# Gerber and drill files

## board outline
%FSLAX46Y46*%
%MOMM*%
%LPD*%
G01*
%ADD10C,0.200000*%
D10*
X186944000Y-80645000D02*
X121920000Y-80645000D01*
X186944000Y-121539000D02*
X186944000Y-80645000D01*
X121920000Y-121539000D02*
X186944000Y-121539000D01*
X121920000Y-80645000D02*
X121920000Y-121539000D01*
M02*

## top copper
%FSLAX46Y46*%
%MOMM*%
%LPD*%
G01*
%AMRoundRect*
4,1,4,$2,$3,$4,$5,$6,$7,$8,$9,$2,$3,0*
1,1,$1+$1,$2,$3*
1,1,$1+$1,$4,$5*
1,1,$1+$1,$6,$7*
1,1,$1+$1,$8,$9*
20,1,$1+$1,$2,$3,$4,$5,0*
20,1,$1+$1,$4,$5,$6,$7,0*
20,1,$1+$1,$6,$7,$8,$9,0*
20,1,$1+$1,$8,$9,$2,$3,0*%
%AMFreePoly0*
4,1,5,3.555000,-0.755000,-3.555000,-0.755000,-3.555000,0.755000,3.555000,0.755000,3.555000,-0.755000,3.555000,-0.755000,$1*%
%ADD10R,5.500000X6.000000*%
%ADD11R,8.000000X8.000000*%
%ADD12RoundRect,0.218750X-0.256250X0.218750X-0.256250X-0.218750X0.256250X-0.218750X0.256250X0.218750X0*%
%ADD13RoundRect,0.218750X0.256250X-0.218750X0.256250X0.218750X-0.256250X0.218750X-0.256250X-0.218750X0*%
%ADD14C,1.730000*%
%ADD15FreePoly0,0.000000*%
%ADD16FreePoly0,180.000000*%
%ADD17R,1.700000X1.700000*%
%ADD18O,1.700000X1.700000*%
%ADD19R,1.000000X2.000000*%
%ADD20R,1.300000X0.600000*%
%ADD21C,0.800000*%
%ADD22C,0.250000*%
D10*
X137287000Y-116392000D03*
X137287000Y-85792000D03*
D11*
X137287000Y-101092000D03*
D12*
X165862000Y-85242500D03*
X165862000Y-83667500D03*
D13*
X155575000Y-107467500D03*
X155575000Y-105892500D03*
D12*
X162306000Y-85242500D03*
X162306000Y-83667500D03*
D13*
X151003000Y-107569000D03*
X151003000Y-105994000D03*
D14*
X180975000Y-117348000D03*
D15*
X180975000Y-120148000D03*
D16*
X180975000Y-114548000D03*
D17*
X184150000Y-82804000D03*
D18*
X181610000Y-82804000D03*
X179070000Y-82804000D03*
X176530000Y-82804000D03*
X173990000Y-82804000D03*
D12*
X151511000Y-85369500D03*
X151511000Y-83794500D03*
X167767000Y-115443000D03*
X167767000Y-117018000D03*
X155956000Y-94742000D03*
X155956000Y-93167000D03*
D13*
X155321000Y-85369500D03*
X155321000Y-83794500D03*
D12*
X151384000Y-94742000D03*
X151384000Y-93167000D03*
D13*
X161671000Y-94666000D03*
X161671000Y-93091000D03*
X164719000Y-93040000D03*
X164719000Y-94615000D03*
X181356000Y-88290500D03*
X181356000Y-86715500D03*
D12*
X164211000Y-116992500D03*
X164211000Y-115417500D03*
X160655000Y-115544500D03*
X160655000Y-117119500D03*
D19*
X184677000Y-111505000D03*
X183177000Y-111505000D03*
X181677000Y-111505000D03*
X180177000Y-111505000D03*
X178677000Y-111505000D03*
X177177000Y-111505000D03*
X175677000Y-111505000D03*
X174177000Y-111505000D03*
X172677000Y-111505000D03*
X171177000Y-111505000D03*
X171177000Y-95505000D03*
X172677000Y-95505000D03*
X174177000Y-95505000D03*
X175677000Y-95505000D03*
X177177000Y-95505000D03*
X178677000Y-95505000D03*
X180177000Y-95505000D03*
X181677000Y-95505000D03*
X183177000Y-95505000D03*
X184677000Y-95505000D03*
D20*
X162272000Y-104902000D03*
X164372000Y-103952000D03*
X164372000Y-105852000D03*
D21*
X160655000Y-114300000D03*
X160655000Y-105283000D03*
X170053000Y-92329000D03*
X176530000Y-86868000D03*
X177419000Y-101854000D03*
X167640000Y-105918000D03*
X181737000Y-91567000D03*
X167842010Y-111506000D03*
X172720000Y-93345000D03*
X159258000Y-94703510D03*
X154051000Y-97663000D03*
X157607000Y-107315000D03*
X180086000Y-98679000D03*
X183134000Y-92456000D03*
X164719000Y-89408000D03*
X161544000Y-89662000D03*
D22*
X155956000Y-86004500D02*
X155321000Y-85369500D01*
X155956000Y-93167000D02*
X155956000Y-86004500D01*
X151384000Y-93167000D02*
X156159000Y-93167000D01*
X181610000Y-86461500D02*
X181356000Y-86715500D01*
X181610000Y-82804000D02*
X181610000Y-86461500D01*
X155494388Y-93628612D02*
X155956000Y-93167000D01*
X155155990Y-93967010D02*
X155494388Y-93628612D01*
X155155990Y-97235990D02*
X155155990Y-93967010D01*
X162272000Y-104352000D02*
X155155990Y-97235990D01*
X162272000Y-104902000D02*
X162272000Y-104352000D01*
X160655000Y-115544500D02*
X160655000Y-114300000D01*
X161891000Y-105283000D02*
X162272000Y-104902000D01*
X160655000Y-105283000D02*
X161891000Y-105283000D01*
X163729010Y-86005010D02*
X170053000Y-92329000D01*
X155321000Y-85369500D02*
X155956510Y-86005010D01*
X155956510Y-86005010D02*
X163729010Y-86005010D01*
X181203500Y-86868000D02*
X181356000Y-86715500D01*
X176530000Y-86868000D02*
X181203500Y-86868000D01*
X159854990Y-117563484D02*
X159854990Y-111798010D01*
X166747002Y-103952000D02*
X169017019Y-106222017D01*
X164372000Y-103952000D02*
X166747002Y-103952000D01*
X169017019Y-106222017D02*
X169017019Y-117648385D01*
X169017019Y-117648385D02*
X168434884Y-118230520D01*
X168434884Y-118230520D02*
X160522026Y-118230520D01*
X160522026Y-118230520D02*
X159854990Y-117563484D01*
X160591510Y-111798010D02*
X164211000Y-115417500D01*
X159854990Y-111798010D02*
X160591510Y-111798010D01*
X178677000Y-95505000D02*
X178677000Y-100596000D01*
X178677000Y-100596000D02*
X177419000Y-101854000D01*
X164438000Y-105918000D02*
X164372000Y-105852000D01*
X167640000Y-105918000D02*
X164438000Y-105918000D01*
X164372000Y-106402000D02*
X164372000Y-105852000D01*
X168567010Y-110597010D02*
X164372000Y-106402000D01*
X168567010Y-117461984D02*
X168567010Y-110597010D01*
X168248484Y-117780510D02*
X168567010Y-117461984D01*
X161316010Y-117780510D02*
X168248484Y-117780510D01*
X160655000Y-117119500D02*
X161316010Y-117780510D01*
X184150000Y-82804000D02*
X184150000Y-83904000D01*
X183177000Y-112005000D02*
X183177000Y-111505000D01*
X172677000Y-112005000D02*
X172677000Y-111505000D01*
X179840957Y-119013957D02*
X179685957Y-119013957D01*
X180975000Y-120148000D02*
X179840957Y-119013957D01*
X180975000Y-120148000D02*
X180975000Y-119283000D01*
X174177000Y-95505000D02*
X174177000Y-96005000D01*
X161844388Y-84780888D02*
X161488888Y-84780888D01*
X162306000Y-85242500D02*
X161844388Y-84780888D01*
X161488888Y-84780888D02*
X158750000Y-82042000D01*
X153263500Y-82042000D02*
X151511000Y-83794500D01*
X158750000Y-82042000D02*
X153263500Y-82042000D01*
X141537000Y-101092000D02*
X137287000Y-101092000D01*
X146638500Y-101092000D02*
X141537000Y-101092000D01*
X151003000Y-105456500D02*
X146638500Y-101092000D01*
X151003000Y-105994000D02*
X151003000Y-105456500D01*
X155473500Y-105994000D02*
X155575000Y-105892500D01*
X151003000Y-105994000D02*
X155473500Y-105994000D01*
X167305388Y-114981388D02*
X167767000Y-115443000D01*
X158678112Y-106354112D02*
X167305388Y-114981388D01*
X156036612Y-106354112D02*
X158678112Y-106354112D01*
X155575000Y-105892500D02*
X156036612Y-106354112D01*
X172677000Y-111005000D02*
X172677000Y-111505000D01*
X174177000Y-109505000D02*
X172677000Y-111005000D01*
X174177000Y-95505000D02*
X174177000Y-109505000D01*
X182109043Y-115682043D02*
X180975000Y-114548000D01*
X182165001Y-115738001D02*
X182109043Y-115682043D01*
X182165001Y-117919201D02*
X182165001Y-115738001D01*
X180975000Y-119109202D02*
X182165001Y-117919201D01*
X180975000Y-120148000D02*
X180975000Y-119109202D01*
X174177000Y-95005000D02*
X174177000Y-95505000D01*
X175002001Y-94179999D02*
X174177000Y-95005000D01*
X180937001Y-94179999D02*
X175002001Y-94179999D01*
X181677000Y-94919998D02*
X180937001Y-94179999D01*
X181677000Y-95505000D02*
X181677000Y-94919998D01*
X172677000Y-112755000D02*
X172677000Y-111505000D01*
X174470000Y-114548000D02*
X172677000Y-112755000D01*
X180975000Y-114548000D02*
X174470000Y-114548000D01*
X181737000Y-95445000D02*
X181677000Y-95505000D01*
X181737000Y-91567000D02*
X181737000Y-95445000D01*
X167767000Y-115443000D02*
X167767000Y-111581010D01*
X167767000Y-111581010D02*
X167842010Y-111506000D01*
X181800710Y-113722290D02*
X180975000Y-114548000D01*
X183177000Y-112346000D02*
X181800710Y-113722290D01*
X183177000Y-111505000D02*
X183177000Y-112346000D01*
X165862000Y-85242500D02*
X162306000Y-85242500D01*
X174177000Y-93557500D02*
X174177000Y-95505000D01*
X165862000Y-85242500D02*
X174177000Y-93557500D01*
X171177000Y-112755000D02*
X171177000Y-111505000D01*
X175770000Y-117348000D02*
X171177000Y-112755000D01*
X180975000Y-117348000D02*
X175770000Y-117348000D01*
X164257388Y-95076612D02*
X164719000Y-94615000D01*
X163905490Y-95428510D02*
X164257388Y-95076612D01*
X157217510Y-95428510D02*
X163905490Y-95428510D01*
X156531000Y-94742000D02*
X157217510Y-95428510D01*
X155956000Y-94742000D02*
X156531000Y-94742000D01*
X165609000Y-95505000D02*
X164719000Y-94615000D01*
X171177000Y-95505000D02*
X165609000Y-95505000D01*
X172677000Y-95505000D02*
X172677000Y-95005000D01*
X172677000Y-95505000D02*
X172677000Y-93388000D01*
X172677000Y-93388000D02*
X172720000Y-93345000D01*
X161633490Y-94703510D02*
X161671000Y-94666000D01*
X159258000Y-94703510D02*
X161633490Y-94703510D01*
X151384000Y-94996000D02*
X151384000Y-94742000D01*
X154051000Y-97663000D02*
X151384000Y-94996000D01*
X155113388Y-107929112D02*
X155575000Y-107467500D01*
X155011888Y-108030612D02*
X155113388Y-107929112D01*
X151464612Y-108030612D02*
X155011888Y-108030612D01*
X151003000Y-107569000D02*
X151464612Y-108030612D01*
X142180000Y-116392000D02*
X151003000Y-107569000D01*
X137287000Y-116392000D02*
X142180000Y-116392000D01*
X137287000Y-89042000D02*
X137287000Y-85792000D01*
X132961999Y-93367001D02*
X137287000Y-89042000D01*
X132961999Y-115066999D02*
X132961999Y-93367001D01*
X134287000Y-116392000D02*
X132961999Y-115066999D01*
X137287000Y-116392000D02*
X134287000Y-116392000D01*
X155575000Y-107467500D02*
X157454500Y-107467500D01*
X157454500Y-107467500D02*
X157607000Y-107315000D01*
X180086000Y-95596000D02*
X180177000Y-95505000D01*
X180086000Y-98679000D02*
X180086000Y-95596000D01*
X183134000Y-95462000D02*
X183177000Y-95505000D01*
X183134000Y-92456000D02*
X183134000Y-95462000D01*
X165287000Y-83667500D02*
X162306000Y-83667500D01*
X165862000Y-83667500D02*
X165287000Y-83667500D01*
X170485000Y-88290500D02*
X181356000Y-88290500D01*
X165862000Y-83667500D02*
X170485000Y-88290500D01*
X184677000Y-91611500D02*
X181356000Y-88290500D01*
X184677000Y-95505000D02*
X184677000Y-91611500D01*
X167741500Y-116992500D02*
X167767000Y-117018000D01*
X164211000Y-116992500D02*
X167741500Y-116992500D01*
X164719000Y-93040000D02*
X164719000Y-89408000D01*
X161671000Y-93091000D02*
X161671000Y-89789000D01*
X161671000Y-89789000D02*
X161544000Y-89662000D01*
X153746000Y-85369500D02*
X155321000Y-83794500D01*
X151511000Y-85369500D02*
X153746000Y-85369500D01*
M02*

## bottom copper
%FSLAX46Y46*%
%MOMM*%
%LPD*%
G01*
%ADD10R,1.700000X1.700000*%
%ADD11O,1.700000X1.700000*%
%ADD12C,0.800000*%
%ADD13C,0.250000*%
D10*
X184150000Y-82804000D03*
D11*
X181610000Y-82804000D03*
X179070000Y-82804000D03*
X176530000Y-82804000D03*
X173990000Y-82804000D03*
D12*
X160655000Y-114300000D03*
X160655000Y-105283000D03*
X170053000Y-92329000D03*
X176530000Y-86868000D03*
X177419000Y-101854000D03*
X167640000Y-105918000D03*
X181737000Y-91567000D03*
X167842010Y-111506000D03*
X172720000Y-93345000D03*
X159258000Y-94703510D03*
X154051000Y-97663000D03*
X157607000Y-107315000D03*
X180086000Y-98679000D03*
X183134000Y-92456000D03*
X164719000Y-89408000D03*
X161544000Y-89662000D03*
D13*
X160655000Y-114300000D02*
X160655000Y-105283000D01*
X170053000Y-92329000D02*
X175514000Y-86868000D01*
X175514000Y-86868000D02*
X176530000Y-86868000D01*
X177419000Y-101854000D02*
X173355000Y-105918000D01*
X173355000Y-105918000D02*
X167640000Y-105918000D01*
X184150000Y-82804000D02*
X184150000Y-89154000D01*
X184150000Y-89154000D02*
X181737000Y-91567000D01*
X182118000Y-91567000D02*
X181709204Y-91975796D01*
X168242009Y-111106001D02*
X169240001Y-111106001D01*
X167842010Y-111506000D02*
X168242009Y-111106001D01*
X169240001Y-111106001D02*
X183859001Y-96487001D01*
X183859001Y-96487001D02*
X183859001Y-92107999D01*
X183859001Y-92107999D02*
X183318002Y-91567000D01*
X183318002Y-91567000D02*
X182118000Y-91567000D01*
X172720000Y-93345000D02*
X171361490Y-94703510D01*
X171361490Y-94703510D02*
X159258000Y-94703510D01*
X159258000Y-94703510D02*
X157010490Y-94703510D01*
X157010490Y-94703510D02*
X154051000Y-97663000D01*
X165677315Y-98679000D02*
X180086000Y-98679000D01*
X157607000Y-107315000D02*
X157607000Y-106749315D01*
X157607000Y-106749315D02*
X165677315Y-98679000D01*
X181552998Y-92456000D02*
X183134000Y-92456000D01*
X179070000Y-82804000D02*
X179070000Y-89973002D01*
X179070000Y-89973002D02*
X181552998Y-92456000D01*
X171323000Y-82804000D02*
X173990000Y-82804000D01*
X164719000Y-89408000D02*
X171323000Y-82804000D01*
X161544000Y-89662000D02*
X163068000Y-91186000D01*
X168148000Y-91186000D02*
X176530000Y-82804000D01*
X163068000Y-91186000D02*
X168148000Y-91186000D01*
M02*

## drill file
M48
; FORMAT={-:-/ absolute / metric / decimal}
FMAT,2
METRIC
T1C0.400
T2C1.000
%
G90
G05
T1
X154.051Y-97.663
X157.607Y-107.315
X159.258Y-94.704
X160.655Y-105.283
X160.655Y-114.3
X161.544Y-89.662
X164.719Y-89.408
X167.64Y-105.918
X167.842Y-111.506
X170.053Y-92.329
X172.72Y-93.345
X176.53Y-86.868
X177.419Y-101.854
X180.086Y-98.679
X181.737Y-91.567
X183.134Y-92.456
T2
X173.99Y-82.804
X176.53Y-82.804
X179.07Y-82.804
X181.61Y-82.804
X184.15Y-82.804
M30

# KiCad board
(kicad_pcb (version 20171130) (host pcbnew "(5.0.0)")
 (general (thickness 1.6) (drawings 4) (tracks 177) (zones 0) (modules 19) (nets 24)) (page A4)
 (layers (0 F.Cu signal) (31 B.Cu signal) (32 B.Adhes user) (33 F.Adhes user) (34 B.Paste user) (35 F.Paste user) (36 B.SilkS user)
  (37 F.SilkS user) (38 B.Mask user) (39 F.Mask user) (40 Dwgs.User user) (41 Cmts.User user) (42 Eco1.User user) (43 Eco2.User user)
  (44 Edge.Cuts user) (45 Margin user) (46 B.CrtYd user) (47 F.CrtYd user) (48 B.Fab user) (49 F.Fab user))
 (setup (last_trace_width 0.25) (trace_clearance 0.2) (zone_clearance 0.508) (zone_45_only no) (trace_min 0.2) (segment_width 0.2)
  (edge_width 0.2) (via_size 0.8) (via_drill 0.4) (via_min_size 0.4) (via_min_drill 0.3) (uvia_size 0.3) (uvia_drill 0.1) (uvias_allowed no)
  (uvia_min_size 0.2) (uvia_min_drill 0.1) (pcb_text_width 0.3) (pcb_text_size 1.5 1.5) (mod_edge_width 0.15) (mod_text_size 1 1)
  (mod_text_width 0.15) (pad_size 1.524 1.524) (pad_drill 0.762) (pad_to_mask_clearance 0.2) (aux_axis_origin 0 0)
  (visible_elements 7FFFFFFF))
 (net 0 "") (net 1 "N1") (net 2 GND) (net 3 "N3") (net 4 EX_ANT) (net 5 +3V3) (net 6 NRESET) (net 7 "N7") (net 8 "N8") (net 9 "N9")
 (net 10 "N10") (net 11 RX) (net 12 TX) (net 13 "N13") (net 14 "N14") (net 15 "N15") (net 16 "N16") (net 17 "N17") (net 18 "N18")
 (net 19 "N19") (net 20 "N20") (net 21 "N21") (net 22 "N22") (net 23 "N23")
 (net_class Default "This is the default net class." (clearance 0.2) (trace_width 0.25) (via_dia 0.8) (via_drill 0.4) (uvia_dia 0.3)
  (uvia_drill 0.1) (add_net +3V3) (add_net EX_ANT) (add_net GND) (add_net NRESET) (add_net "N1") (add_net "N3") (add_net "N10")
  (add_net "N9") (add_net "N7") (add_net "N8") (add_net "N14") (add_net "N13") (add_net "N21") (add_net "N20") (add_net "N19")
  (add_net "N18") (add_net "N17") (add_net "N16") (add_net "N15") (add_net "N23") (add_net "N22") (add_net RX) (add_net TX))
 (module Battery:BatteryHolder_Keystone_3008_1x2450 (layer F.Cu) (at 137.287 101.092 90)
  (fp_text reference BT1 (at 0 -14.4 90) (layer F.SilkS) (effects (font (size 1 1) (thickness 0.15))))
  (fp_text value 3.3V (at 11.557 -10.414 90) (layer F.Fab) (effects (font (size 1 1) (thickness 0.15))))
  (pad 1 smd rect (at -15.3 0 90) (size 6 5.5) (layers F.Cu F.Paste F.Mask) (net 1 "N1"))
  (pad 1 smd rect (at 15.3 0 90) (size 6 5.5) (layers F.Cu F.Paste F.Mask) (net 1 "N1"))
  (pad 2 smd rect (at 0 0 90) (size 8 8) (layers F.Cu F.Mask) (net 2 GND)))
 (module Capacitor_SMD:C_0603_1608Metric (layer F.Cu) (at 165.862 84.455 270)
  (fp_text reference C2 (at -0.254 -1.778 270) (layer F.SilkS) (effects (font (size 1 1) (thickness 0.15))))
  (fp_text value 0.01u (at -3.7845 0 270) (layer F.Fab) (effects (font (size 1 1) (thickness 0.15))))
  (pad 2 smd roundrect (at 0.7875 0 270) (size 0.875 0.95) (layers F.Cu F.Paste F.Mask) (roundrect_rratio 0.25) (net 2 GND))
  (pad 1 smd roundrect (at -0.7875 0 270) (size 0.875 0.95) (layers F.Cu F.Paste F.Mask) (roundrect_rratio 0.25) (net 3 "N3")))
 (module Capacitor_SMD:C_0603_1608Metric (layer F.Cu) (at 155.575 106.68 90)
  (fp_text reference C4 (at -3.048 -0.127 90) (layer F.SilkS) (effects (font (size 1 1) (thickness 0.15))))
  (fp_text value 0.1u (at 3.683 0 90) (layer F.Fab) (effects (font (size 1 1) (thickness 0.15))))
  (pad 1 smd roundrect (at -0.7875 0 90) (size 0.875 0.95) (layers F.Cu F.Paste F.Mask) (roundrect_rratio 0.25) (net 1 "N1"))
  (pad 2 smd roundrect (at 0.7875 0 90) (size 0.875 0.95) (layers F.Cu F.Paste F.Mask) (roundrect_rratio 0.25) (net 2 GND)))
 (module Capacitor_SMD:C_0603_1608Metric (layer F.Cu) (at 162.306 84.455 270)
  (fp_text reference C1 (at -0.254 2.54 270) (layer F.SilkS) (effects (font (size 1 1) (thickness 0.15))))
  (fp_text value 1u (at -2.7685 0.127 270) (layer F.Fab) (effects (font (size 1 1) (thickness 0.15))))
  (pad 2 smd roundrect (at 0.7875 0 270) (size 0.875 0.95) (layers F.Cu F.Paste F.Mask) (roundrect_rratio 0.25) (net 2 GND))
  (pad 1 smd roundrect (at -0.7875 0 270) (size 0.875 0.95) (layers F.Cu F.Paste F.Mask) (roundrect_rratio 0.25) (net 3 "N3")))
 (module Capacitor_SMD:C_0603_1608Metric (layer F.Cu) (at 151.003 106.7815 90)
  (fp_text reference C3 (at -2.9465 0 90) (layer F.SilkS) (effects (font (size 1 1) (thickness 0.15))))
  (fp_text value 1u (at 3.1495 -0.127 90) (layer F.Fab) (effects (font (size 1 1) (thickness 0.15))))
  (pad 1 smd roundrect (at -0.7875 0 90) (size 0.875 0.95) (layers F.Cu F.Paste F.Mask) (roundrect_rratio 0.25) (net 1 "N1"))
  (pad 2 smd roundrect (at 0.7875 0 90) (size 0.875 0.95) (layers F.Cu F.Paste F.Mask) (roundrect_rratio 0.25) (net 2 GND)))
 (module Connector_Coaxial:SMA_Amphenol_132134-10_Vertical (layer F.Cu) (at 180.975 117.348)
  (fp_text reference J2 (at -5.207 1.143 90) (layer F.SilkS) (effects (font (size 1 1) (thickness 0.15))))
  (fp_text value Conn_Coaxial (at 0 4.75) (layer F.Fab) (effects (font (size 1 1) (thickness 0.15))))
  (pad 1 smd circle (at 0 0 90) (size 1.73 1.73) (layers F.Cu F.Paste F.Mask) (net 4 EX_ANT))
  (pad 2 smd custom (at 0 2.8) (size 7.11 1.51) (layers F.Cu F.Paste F.Mask) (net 2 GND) (zone_connect 2)
   (options (clearance outline) (anchor rect)) (primitives))
  (pad 2 smd custom (at 0 -2.8 180) (size 7.11 1.51) (layers F.Cu F.Paste F.Mask) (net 2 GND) (zone_connect 2)
   (options (clearance outline) (anchor rect)) (primitives)))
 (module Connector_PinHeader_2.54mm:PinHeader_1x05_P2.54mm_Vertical (layer F.Cu) (at 184.15 82.804 270)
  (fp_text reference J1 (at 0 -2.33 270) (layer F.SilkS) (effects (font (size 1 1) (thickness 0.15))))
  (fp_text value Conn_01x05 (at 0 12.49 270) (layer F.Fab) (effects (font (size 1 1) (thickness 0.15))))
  (pad 1 thru_hole rect (at 0 0 270) (size 1.7 1.7) (drill 1) (layers *.Cu *.Mask) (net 2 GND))
  (pad 2 thru_hole oval (at 0 2.54 270) (size 1.7 1.7) (drill 1) (layers *.Cu *.Mask) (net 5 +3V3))
  (pad 3 thru_hole oval (at 0 5.08 270) (size 1.7 1.7) (drill 1) (layers *.Cu *.Mask) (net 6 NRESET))
  (pad 4 thru_hole oval (at 0 7.62 270) (size 1.7 1.7) (drill 1) (layers *.Cu *.Mask) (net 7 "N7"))
  (pad 5 thru_hole oval (at 0 10.16 270) (size 1.7 1.7) (drill 1) (layers *.Cu *.Mask) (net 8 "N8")))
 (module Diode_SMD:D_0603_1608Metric (layer F.Cu) (at 151.511 84.582 270)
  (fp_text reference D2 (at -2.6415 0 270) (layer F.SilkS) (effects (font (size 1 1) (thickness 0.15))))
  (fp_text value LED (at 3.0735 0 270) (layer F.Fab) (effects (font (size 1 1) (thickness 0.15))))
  (pad 2 smd roundrect (at 0.7875 0 270) (size 0.875 0.95) (layers F.Cu F.Paste F.Mask) (roundrect_rratio 0.25) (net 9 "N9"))
  (pad 1 smd roundrect (at -0.7875 0 270) (size 0.875 0.95) (layers F.Cu F.Paste F.Mask) (roundrect_rratio 0.25) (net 2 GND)))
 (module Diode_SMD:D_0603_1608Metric (layer F.Cu) (at 167.767 116.2305 270)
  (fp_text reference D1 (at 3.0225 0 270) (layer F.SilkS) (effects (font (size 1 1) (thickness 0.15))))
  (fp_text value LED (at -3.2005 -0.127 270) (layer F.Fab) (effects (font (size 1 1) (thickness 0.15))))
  (pad 1 smd roundrect (at -0.7875 0 270) (size 0.875 0.95) (layers F.Cu F.Paste F.Mask) (roundrect_rratio 0.25) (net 2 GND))
  (pad 2 smd roundrect (at 0.7875 0 270) (size 0.875 0.95) (layers F.Cu F.Paste F.Mask) (roundrect_rratio 0.25) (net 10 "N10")))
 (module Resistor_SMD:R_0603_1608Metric (layer F.Cu) (at 155.956 93.9545 270)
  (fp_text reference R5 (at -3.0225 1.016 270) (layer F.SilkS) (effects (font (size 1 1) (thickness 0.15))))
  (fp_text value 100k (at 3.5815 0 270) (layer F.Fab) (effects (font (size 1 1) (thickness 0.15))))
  (pad 2 smd roundrect (at 0.7875 0 270) (size 0.875 0.95) (layers F.Cu F.Paste F.Mask) (roundrect_rratio 0.25) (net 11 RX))
  (pad 1 smd roundrect (at -0.7875 0 270) (size 0.875 0.95) (layers F.Cu F.Paste F.Mask) (roundrect_rratio 0.25) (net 5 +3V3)))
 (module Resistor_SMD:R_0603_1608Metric (layer F.Cu) (at 155.321 84.582 90)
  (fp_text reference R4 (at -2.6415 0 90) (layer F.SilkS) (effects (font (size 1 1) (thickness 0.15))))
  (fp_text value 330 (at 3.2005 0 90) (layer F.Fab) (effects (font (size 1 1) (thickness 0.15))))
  (pad 1 smd roundrect (at -0.7875 0 90) (size 0.875 0.95) (layers F.Cu F.Paste F.Mask) (roundrect_rratio 0.25) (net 5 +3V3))
  (pad 2 smd roundrect (at 0.7875 0 90) (size 0.875 0.95) (layers F.Cu F.Paste F.Mask) (roundrect_rratio 0.25) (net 9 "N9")))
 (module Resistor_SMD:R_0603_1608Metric (layer F.Cu) (at 151.384 93.9545 270)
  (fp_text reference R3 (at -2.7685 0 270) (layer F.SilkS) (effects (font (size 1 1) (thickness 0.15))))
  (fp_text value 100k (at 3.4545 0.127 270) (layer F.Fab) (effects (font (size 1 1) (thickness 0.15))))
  (pad 2 smd roundrect (at 0.7875 0 270) (size 0.875 0.95) (layers F.Cu F.Paste F.Mask) (roundrect_rratio 0.25) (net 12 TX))
  (pad 1 smd roundrect (at -0.7875 0 270) (size 0.875 0.95) (layers F.Cu F.Paste F.Mask) (roundrect_rratio 0.25) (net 5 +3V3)))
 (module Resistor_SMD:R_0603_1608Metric (layer F.Cu) (at 161.671 93.8785 90)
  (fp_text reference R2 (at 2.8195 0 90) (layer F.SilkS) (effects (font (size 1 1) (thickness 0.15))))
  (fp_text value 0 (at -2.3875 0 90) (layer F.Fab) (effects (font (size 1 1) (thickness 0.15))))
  (pad 1 smd roundrect (at -0.7875 0 90) (size 0.875 0.95) (layers F.Cu F.Paste F.Mask) (roundrect_rratio 0.25) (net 12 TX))
  (pad 2 smd roundrect (at 0.7875 0 90) (size 0.875 0.95) (layers F.Cu F.Paste F.Mask) (roundrect_rratio 0.25) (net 7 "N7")))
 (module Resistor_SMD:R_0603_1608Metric (layer F.Cu) (at 164.719 93.8275 90)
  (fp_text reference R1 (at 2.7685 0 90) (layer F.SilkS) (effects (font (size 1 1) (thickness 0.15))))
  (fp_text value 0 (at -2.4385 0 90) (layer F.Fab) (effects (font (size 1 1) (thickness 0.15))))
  (pad 2 smd roundrect (at 0.7875 0 90) (size 0.875 0.95) (layers F.Cu F.Paste F.Mask) (roundrect_rratio 0.25) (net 8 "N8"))
  (pad 1 smd roundrect (at -0.7875 0 90) (size 0.875 0.95) (layers F.Cu F.Paste F.Mask) (roundrect_rratio 0.25) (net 11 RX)))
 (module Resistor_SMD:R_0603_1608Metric (layer F.Cu) (at 181.356 87.503 90)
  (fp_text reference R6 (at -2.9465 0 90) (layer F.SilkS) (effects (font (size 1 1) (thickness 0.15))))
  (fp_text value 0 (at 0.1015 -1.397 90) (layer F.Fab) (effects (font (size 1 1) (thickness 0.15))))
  (pad 1 smd roundrect (at -0.7875 0 90) (size 0.875 0.95) (layers F.Cu F.Paste F.Mask) (roundrect_rratio 0.25) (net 3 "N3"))
  (pad 2 smd roundrect (at 0.7875 0 90) (size 0.875 0.95) (layers F.Cu F.Paste F.Mask) (roundrect_rratio 0.25) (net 5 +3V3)))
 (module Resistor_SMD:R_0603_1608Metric (layer F.Cu) (at 164.211 116.205 270)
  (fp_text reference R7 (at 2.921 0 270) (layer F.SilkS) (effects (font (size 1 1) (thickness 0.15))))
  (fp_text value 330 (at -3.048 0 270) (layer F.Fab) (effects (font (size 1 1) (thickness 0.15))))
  (pad 2 smd roundrect (at 0.7875 0 270) (size 0.875 0.95) (layers F.Cu F.Paste F.Mask) (roundrect_rratio 0.25) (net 10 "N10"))
  (pad 1 smd roundrect (at -0.7875 0 270) (size 0.875 0.95) (layers F.Cu F.Paste F.Mask) (roundrect_rratio 0.25) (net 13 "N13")))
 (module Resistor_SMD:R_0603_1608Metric (layer F.Cu) (at 160.655 116.332 270)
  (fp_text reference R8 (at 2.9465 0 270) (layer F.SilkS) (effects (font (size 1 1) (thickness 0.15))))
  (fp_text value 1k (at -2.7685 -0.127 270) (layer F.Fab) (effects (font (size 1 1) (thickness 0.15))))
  (pad 1 smd roundrect (at -0.7875 0 270) (size 0.875 0.95) (layers F.Cu F.Paste F.Mask) (roundrect_rratio 0.25) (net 5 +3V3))
  (pad 2 smd roundrect (at 0.7875 0 270) (size 0.875 0.95) (layers F.Cu F.Paste F.Mask) (roundrect_rratio 0.25) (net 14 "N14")))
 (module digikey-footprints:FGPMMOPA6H (layer F.Cu) (at 177.927 103.505 270)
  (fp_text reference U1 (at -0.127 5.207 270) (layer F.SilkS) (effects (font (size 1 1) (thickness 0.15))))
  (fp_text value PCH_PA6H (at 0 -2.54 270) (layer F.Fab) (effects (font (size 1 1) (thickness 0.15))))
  (pad 20 smd rect (at 8 -6.75 270) (size 2 1) (layers F.Cu F.Paste F.Mask) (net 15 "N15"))
  (pad 19 smd rect (at 8 -5.25 270) (size 2 1) (layers F.Cu F.Paste F.Mask) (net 2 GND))
  (pad 18 smd rect (at 8 -3.75 270) (size 2 1) (layers F.Cu F.Paste F.Mask) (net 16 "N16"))
  (pad 17 smd rect (at 8 -2.25 270) (size 2 1) (layers F.Cu F.Paste F.Mask) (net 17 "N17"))
  (pad 16 smd rect (at 8 -0.75 270) (size 2 1) (layers F.Cu F.Paste F.Mask) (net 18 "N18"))
  (pad 15 smd rect (at 8 0.75 270) (size 2 1) (layers F.Cu F.Paste F.Mask) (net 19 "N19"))
  (pad 14 smd rect (at 8 2.25 270) (size 2 1) (layers F.Cu F.Paste F.Mask) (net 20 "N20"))
  (pad 13 smd rect (at 8 3.75 270) (size 2 1) (layers F.Cu F.Paste F.Mask) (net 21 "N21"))
  (pad 12 smd rect (at 8 5.25 270) (size 2 1) (layers F.Cu F.Paste F.Mask) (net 2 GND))
  (pad 11 smd rect (at 8 6.75 270) (size 2 1) (layers F.Cu F.Paste F.Mask) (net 4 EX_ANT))
  (pad 10 smd rect (at -8 6.75 270) (size 2 1) (layers F.Cu F.Paste F.Mask) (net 11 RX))
  (pad 9 smd rect (at -8 5.25 270) (size 2 1) (layers F.Cu F.Paste F.Mask) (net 12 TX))
  (pad 8 smd rect (at -8 3.75 270) (size 2 1) (layers F.Cu F.Paste F.Mask) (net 2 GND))
  (pad 7 smd rect (at -8 2.25 270) (size 2 1) (layers F.Cu F.Paste F.Mask) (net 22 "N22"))
  (pad 6 smd rect (at -8 0.75 270) (size 2 1) (layers F.Cu F.Paste F.Mask) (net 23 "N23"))
  (pad 5 smd rect (at -8 -0.75 270) (size 2 1) (layers F.Cu F.Paste F.Mask) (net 14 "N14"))
  (pad 4 smd rect (at -8 -2.25 270) (size 2 1) (layers F.Cu F.Paste F.Mask) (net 1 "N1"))
  (pad 3 smd rect (at -8 -3.75 270) (size 2 1) (layers F.Cu F.Paste F.Mask) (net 2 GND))
  (pad 2 smd rect (at -8 -5.25 270) (size 2 1) (layers F.Cu F.Paste F.Mask) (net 6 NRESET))
  (pad 1 smd rect (at -8 -6.75 270) (size 2 1) (layers F.Cu F.Paste F.Mask) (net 3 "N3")))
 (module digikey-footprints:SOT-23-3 (layer F.Cu) (at 163.322 104.902 180)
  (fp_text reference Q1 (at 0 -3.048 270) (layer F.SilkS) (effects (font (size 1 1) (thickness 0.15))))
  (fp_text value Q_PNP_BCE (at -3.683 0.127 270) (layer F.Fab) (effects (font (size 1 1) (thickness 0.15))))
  (pad 3 smd rect (at 1.05 0 180) (size 1.3 0.6) (layers F.Cu F.Paste F.Mask) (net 5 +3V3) (solder_mask_margin 0.07))
  (pad 2 smd rect (at -1.05 0.95 180) (size 1.3 0.6) (layers F.Cu F.Paste F.Mask) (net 13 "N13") (solder_mask_margin 0.07))
  (pad 1 smd rect (at -1.05 -0.95 180) (size 1.3 0.6) (layers F.Cu F.Paste F.Mask) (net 14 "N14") (solder_mask_margin 0.07)))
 (gr_line (start 186.944 80.645) (end 121.92 80.645) (layer Edge.Cuts) (width 0.2))
 (gr_line (start 186.944 121.539) (end 186.944 80.645) (layer Edge.Cuts) (width 0.2))
 (gr_line (start 121.92 121.539) (end 186.944 121.539) (layer Edge.Cuts) (width 0.2))
 (gr_line (start 121.92 80.645) (end 121.92 121.539) (layer Edge.Cuts) (width 0.2))
 (segment (start 155.956 86.0045) (end 155.321 85.3695) (width 0.25) (layer F.Cu) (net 5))
 (segment (start 155.956 93.167) (end 155.956 86.0045) (width 0.25) (layer F.Cu) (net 5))
 (segment (start 151.384 93.167) (end 156.159 93.167) (width 0.25) (layer F.Cu) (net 5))
 (segment (start 181.61 86.4615) (end 181.356 86.7155) (width 0.25) (layer F.Cu) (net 5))
 (segment (start 181.61 82.804) (end 181.61 86.4615) (width 0.25) (layer F.Cu) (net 5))
 (segment (start 155.494388 93.628612) (end 155.956 93.167) (width 0.25) (layer F.Cu) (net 5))
 (segment (start 155.15599 93.96701) (end 155.494388 93.628612) (width 0.25) (layer F.Cu) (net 5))
 (segment (start 155.15599 97.23599) (end 155.15599 93.96701) (width 0.25) (layer F.Cu) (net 5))
 (segment (start 162.272 104.352) (end 155.15599 97.23599) (width 0.25) (layer F.Cu) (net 5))
 (segment (start 162.272 104.902) (end 162.272 104.352) (width 0.25) (layer F.Cu) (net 5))
 (via (at 160.655 114.3) (size 0.8) (drill 0.4) (layers F.Cu B.Cu) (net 5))
 (segment (start 160.655 115.5445) (end 160.655 114.3) (width 0.25) (layer F.Cu) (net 5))
 (via (at 160.655 105.283) (size 0.8) (drill 0.4) (layers F.Cu B.Cu) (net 5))
 (segment (start 160.655 114.3) (end 160.655 105.283) (width 0.25) (layer B.Cu) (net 5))
 (segment (start 161.891 105.283) (end 162.272 104.902) (width 0.25) (layer F.Cu) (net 5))
 (segment (start 160.655 105.283) (end 161.891 105.283) (width 0.25) (layer F.Cu) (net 5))
 (via (at 170.053 92.329) (size 0.8) (drill 0.4) (layers F.Cu B.Cu) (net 5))
 (segment (start 163.72901 86.00501) (end 170.053 92.329) (width 0.25) (layer F.Cu) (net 5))
 (segment (start 155.321 85.3695) (end 155.95651 86.00501) (width 0.25) (layer F.Cu) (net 5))
 (segment (start 155.95651 86.00501) (end 163.72901 86.00501) (width 0.25) (layer F.Cu) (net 5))
 (via (at 176.53 86.868) (size 0.8) (drill 0.4) (layers F.Cu B.Cu) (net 5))
 (segment (start 170.053 92.329) (end 175.514 86.868) (width 0.25) (layer B.Cu) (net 5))
 (segment (start 175.514 86.868) (end 176.53 86.868) (width 0.25) (layer B.Cu) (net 5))
 (segment (start 181.2035 86.868) (end 181.356 86.7155) (width 0.25) (layer F.Cu) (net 5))
 (segment (start 176.53 86.868) (end 181.2035 86.868) (width 0.25) (layer F.Cu) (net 5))
 (segment (start 159.85499 117.563484) (end 159.85499 111.79801) (width 0.25) (layer F.Cu) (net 13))
 (segment (start 166.747002 103.952) (end 169.017019 106.222017) (width 0.25) (layer F.Cu) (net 13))
 (segment (start 164.372 103.952) (end 166.747002 103.952) (width 0.25) (layer F.Cu) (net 13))
 (segment (start 169.017019 106.222017) (end 169.017019 117.648385) (width 0.25) (layer F.Cu) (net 13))
 (segment (start 169.017019 117.648385) (end 168.434884 118.23052) (width 0.25) (layer F.Cu) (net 13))
 (segment (start 168.434884 118.23052) (end 160.522026 118.23052) (width 0.25) (layer F.Cu) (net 13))
 (segment (start 160.522026 118.23052) (end 159.85499 117.563484) (width 0.25) (layer F.Cu) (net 13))
 (segment (start 160.59151 111.79801) (end 164.211 115.4175) (width 0.25) (layer F.Cu) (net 13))
 (segment (start 159.85499 111.79801) (end 160.59151 111.79801) (width 0.25) (layer F.Cu) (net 13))
 (via (at 177.419 101.854) (size 0.8) (drill 0.4) (layers F.Cu B.Cu) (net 14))
 (segment (start 178.677 95.505) (end 178.677 100.596) (width 0.25) (layer F.Cu) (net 14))
 (segment (start 178.677 100.596) (end 177.419 101.854) (width 0.25) (layer F.Cu) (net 14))
 (via (at 167.64 105.918) (size 0.8) (drill 0.4) (layers F.Cu B.Cu) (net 14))
 (segment (start 177.419 101.854) (end 173.355 105.918) (width 0.25) (layer B.Cu) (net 14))
 (segment (start 173.355 105.918) (end 167.64 105.918) (width 0.25) (layer B.Cu) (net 14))
 (segment (start 164.438 105.918) (end 164.372 105.852) (width 0.25) (layer F.Cu) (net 14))
 (segment (start 167.64 105.918) (end 164.438 105.918) (width 0.25) (layer F.Cu) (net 14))
 (segment (start 164.372 106.402) (end 164.372 105.852) (width 0.25) (layer F.Cu) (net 14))
 (segment (start 168.56701 110.59701) (end 164.372 106.402) (width 0.25) (layer F.Cu) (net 14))
 (segment (start 168.56701 117.461984) (end 168.56701 110.59701) (width 0.25) (layer F.Cu) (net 14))
 (segment (start 168.248484 117.78051) (end 168.56701 117.461984) (width 0.25) (layer F.Cu) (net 14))
 (segment (start 161.31601 117.78051) (end 168.248484 117.78051) (width 0.25) (layer F.Cu) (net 14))
 (segment (start 160.655 117.1195) (end 161.31601 117.78051) (width 0.25) (layer F.Cu) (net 14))
 (segment (start 184.15 82.804) (end 184.15 83.904) (width 0.25) (layer F.Cu) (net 2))
 (segment (start 183.177 112.005) (end 183.177 111.505) (width 0.25) (layer F.Cu) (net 2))
 (segment (start 172.677 112.005) (end 172.677 111.505) (width 0.25) (layer F.Cu) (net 2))
 (segment (start 179.840957 119.013957) (end 179.685957 119.013957) (width 0.25) (layer F.Cu) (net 2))
 (segment (start 180.975 120.148) (end 179.840957 119.013957) (width 0.25) (layer F.Cu) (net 2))
 (segment (start 180.975 120.148) (end 180.975 119.283) (width 0.25) (layer F.Cu) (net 2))
 (segment (start 174.177 95.505) (end 174.177 96.005) (width 0.25) (layer F.Cu) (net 2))
 (segment (start 161.844388 84.780888) (end 161.488888 84.780888) (width 0.25) (layer F.Cu) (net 2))
 (segment (start 162.306 85.2425) (end 161.844388 84.780888) (width 0.25) (layer F.Cu) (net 2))
 (segment (start 161.488888 84.780888) (end 158.75 82.042) (width 0.25) (layer F.Cu) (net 2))
 (segment (start 153.2635 82.042) (end 151.511 83.7945) (width 0.25) (layer F.Cu) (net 2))
 (segment (start 158.75 82.042) (end 153.2635 82.042) (width 0.25) (layer F.Cu) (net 2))
 (segment (start 141.537 101.092) (end 137.287 101.092) (width 0.25) (layer F.Cu) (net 2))
 (segment (start 146.6385 101.092) (end 141.537 101.092) (width 0.25) (layer F.Cu) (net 2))
 (segment (start 151.003 105.4565) (end 146.6385 101.092) (width 0.25) (layer F.Cu) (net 2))
 (segment (start 151.003 105.994) (end 151.003 105.4565) (width 0.25) (layer F.Cu) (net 2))
 (segment (start 155.4735 105.994) (end 155.575 105.8925) (width 0.25) (layer F.Cu) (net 2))
 (segment (start 151.003 105.994) (end 155.4735 105.994) (width 0.25) (layer F.Cu) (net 2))
 (segment (start 167.305388 114.981388) (end 167.767 115.443) (width 0.25) (layer F.Cu) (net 2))
 (segment (start 158.678112 106.354112) (end 167.305388 114.981388) (width 0.25) (layer F.Cu) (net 2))
 (segment (start 156.036612 106.354112) (end 158.678112 106.354112) (width 0.25) (layer F.Cu) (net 2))
 (segment (start 155.575 105.8925) (end 156.036612 106.354112) (width 0.25) (layer F.Cu) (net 2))
 (segment (start 172.677 111.005) (end 172.677 111.505) (width 0.25) (layer F.Cu) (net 2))
 (segment (start 174.177 109.505) (end 172.677 111.005) (width 0.25) (layer F.Cu) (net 2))
 (segment (start 174.177 95.505) (end 174.177 109.505) (width 0.25) (layer F.Cu) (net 2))
 (segment (start 182.109043 115.682043) (end 180.975 114.548) (width 0.25) (layer F.Cu) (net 2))
 (segment (start 182.165001 115.738001) (end 182.109043 115.682043) (width 0.25) (layer F.Cu) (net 2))
 (segment (start 182.165001 117.919201) (end 182.165001 115.738001) (width 0.25) (layer F.Cu) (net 2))
 (segment (start 180.975 119.109202) (end 182.165001 117.919201) (width 0.25) (layer F.Cu) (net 2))
 (segment (start 180.975 120.148) (end 180.975 119.109202) (width 0.25) (layer F.Cu) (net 2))
 (segment (start 174.177 95.005) (end 174.177 95.505) (width 0.25) (layer F.Cu) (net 2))
 (segment (start 175.002001 94.179999) (end 174.177 95.005) (width 0.25) (layer F.Cu) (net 2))
 (segment (start 180.937001 94.179999) (end 175.002001 94.179999) (width 0.25) (layer F.Cu) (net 2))
 (segment (start 181.677 94.919998) (end 180.937001 94.179999) (width 0.25) (layer F.Cu) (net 2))
 (segment (start 181.677 95.505) (end 181.677 94.919998) (width 0.25) (layer F.Cu) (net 2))
 (segment (start 172.677 112.755) (end 172.677 111.505) (width 0.25) (layer F.Cu) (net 2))
 (segment (start 174.47 114.548) (end 172.677 112.755) (width 0.25) (layer F.Cu) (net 2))
 (segment (start 180.975 114.548) (end 174.47 114.548) (width 0.25) (layer F.Cu) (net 2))
 (via (at 181.737 91.567) (size 0.8) (drill 0.4) (layers F.Cu B.Cu) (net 2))
 (segment (start 184.15 82.804) (end 184.15 89.154) (width 0.25) (layer B.Cu) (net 2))
 (segment (start 184.15 89.154) (end 181.737 91.567) (width 0.25) (layer B.Cu) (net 2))
 (segment (start 181.737 95.445) (end 181.677 95.505) (width 0.25) (layer F.Cu) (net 2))
 (segment (start 181.737 91.567) (end 181.737 95.445) (width 0.25) (layer F.Cu) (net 2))
 (via (at 167.84201 111.506) (size 0.8) (drill 0.4) (layers F.Cu B.Cu) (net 2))
 (segment (start 167.767 115.443) (end 167.767 111.58101) (width 0.25) (layer F.Cu) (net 2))
 (segment (start 167.767 111.58101) (end 167.84201 111.506) (width 0.25) (layer F.Cu) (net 2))
 (segment (start 182.118 91.567) (end 181.709204 91.975796) (width 0.25) (layer B.Cu) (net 2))
 (segment (start 168.242009 111.106001) (end 169.240001 111.106001) (width 0.25) (layer B.Cu) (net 2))
 (segment (start 167.84201 111.506) (end 168.242009 111.106001) (width 0.25) (layer B.Cu) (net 2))
 (segment (start 169.240001 111.106001) (end 183.859001 96.487001) (width 0.25) (layer B.Cu) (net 2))
 (segment (start 183.859001 96.487001) (end 183.859001 92.107999) (width 0.25) (layer B.Cu) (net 2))
 (segment (start 183.859001 92.107999) (end 183.318002 91.567) (width 0.25) (layer B.Cu) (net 2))
 (segment (start 183.318002 91.567) (end 182.118 91.567) (width 0.25) (layer B.Cu) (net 2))
 (segment (start 181.80071 113.72229) (end 180.975 114.548) (width 0.25) (layer F.Cu) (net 2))
 (segment (start 183.177 112.346) (end 181.80071 113.72229) (width 0.25) (layer F.Cu) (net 2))
 (segment (start 183.177 111.505) (end 183.177 112.346) (width 0.25) (layer F.Cu) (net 2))
 (segment (start 165.862 85.2425) (end 162.306 85.2425) (width 0.25) (layer F.Cu) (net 2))
 (segment (start 174.177 93.5575) (end 174.177 95.505) (width 0.25) (layer F.Cu) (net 2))
 (segment (start 165.862 85.2425) (end 174.177 93.5575) (width 0.25) (layer F.Cu) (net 2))
 (segment (start 171.177 112.755) (end 171.177 111.505) (width 0.25) (layer F.Cu) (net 4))
 (segment (start 175.77 117.348) (end 171.177 112.755) (width 0.25) (layer F.Cu) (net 4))
 (segment (start 180.975 117.348) (end 175.77 117.348) (width 0.25) (layer F.Cu) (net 4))
 (segment (start 164.257388 95.076612) (end 164.719 94.615) (width 0.25) (layer F.Cu) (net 11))
 (segment (start 163.90549 95.42851) (end 164.257388 95.076612) (width 0.25) (layer F.Cu) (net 11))
 (segment (start 157.21751 95.42851) (end 163.90549 95.42851) (width 0.25) (layer F.Cu) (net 11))
 (segment (start 156.531 94.742) (end 157.21751 95.42851) (width 0.25) (layer F.Cu) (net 11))
 (segment (start 155.956 94.742) (end 156.531 94.742) (width 0.25) (layer F.Cu) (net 11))
 (segment (start 165.609 95.505) (end 164.719 94.615) (width 0.25) (layer F.Cu) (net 11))
 (segment (start 171.177 95.505) (end 165.609 95.505) (width 0.25) (layer F.Cu) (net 11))
 (segment (start 172.677 95.505) (end 172.677 95.005) (width 0.25) (layer F.Cu) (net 12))
 (via (at 172.72 93.345) (size 0.8) (drill 0.4) (layers F.Cu B.Cu) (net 12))
 (segment (start 172.677 95.505) (end 172.677 93.388) (width 0.25) (layer F.Cu) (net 12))
 (segment (start 172.677 93.388) (end 172.72 93.345) (width 0.25) (layer F.Cu) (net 12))
 (via (at 159.258 94.70351) (size 0.8) (drill 0.4) (layers F.Cu B.Cu) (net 12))
 (segment (start 172.72 93.345) (end 171.36149 94.70351) (width 0.25) (layer B.Cu) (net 12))
 (segment (start 171.36149 94.70351) (end 159.258 94.70351) (width 0.25) (layer B.Cu) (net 12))
 (segment (start 161.63349 94.70351) (end 161.671 94.666) (width 0.25) (layer F.Cu) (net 12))
 (segment (start 159.258 94.70351) (end 161.63349 94.70351) (width 0.25) (layer F.Cu) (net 12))
 (via (at 154.051 97.663) (size 0.8) (drill 0.4) (layers F.Cu B.Cu) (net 12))
 (segment (start 159.258 94.70351) (end 157.01049 94.70351) (width 0.25) (layer B.Cu) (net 12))
 (segment (start 157.01049 94.70351) (end 154.051 97.663) (width 0.25) (layer B.Cu) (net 12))
 (segment (start 151.384 94.996) (end 151.384 94.742) (width 0.25) (layer F.Cu) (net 12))
 (segment (start 154.051 97.663) (end 151.384 94.996) (width 0.25) (layer F.Cu) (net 12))
 (segment (start 155.113388 107.929112) (end 155.575 107.4675) (width 0.25) (layer F.Cu) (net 1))
 (segment (start 155.011888 108.030612) (end 155.113388 107.929112) (width 0.25) (layer F.Cu) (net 1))
 (segment (start 151.464612 108.030612) (end 155.011888 108.030612) (width 0.25) (layer F.Cu) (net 1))
 (segment (start 151.003 107.569) (end 151.464612 108.030612) (width 0.25) (layer F.Cu) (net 1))
 (segment (start 142.18 116.392) (end 151.003 107.569) (width 0.25) (layer F.Cu) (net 1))
 (segment (start 137.287 116.392) (end 142.18 116.392) (width 0.25) (layer F.Cu) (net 1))
 (segment (start 137.287 89.042) (end 137.287 85.792) (width 0.25) (layer F.Cu) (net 1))
 (segment (start 132.961999 93.367001) (end 137.287 89.042) (width 0.25) (layer F.Cu) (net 1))
 (segment (start 132.961999 115.066999) (end 132.961999 93.367001) (width 0.25) (layer F.Cu) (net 1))
 (segment (start 134.287 116.392) (end 132.961999 115.066999) (width 0.25) (layer F.Cu) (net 1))
 (segment (start 137.287 116.392) (end 134.287 116.392) (width 0.25) (layer F.Cu) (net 1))
 (via (at 157.607 107.315) (size 0.8) (drill 0.4) (layers F.Cu B.Cu) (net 1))
 (segment (start 155.575 107.4675) (end 157.4545 107.4675) (width 0.25) (layer F.Cu) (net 1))
 (segment (start 157.4545 107.4675) (end 157.607 107.315) (width 0.25) (layer F.Cu) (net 1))
 (via (at 180.086 98.679) (size 0.8) (drill 0.4) (layers F.Cu B.Cu) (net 1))
 (segment (start 165.677315 98.679) (end 180.086 98.679) (width 0.25) (layer B.Cu) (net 1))
 (segment (start 157.607 107.315) (end 157.607 106.749315) (width 0.25) (layer B.Cu) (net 1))
 (segment (start 157.607 106.749315) (end 165.677315 98.679) (width 0.25) (layer B.Cu) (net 1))
 (segment (start 180.086 95.596) (end 180.177 95.505) (width 0.25) (layer F.Cu) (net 1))
 (segment (start 180.086 98.679) (end 180.086 95.596) (width 0.25) (layer F.Cu) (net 1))
 (via (at 183.134 92.456) (size 0.8) (drill 0.4) (layers F.Cu B.Cu) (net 6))
 (segment (start 181.552998 92.456) (end 183.134 92.456) (width 0.25) (layer B.Cu) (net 6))
 (segment (start 179.07 82.804) (end 179.07 89.973002) (width 0.25) (layer B.Cu) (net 6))
 (segment (start 179.07 89.973002) (end 181.552998 92.456) (width 0.25) (layer B.Cu) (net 6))
 (segment (start 183.134 95.462) (end 183.177 95.505) (width 0.25) (layer F.Cu) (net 6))
 (segment (start 183.134 92.456) (end 183.134 95.462) (width 0.25) (layer F.Cu) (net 6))
 (segment (start 165.287 83.6675) (end 162.306 83.6675) (width 0.25) (layer F.Cu) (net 3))
 (segment (start 165.862 83.6675) (end 165.287 83.6675) (width 0.25) (layer F.Cu) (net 3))
 (segment (start 170.485 88.2905) (end 181.356 88.2905) (width 0.25) (layer F.Cu) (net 3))
 (segment (start 165.862 83.6675) (end 170.485 88.2905) (width 0.25) (layer F.Cu) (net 3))
 (segment (start 184.677 91.6115) (end 181.356 88.2905) (width 0.25) (layer F.Cu) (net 3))
 (segment (start 184.677 95.505) (end 184.677 91.6115) (width 0.25) (layer F.Cu) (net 3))
 (segment (start 167.7415 116.9925) (end 167.767 117.018) (width 0.25) (layer F.Cu) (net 10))
 (segment (start 164.211 116.9925) (end 167.7415 116.9925) (width 0.25) (layer F.Cu) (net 10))
 (via (at 164.719 89.408) (size 0.8) (drill 0.4) (layers F.Cu B.Cu) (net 8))
 (segment (start 164.719 93.04) (end 164.719 89.408) (width 0.25) (layer F.Cu) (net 8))
 (segment (start 171.323 82.804) (end 173.99 82.804) (width 0.25) (layer B.Cu) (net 8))
 (segment (start 164.719 89.408) (end 171.323 82.804) (width 0.25) (layer B.Cu) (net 8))
 (via (at 161.544 89.662) (size 0.8) (drill 0.4) (layers F.Cu B.Cu) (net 7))
 (segment (start 161.671 93.091) (end 161.671 89.789) (width 0.25) (layer F.Cu) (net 7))
 (segment (start 161.671 89.789) (end 161.544 89.662) (width 0.25) (layer F.Cu) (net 7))
 (segment (start 161.544 89.662) (end 163.068 91.186) (width 0.25) (layer B.Cu) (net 7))
 (segment (start 168.148 91.186) (end 176.53 82.804) (width 0.25) (layer B.Cu) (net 7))
 (segment (start 163.068 91.186) (end 168.148 91.186) (width 0.25) (layer B.Cu) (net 7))
 (segment (start 153.746 85.3695) (end 155.321 83.7945) (width 0.25) (layer F.Cu) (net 9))
 (segment (start 151.511 85.3695) (end 153.746 85.3695) (width 0.25) (layer F.Cu) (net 9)))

